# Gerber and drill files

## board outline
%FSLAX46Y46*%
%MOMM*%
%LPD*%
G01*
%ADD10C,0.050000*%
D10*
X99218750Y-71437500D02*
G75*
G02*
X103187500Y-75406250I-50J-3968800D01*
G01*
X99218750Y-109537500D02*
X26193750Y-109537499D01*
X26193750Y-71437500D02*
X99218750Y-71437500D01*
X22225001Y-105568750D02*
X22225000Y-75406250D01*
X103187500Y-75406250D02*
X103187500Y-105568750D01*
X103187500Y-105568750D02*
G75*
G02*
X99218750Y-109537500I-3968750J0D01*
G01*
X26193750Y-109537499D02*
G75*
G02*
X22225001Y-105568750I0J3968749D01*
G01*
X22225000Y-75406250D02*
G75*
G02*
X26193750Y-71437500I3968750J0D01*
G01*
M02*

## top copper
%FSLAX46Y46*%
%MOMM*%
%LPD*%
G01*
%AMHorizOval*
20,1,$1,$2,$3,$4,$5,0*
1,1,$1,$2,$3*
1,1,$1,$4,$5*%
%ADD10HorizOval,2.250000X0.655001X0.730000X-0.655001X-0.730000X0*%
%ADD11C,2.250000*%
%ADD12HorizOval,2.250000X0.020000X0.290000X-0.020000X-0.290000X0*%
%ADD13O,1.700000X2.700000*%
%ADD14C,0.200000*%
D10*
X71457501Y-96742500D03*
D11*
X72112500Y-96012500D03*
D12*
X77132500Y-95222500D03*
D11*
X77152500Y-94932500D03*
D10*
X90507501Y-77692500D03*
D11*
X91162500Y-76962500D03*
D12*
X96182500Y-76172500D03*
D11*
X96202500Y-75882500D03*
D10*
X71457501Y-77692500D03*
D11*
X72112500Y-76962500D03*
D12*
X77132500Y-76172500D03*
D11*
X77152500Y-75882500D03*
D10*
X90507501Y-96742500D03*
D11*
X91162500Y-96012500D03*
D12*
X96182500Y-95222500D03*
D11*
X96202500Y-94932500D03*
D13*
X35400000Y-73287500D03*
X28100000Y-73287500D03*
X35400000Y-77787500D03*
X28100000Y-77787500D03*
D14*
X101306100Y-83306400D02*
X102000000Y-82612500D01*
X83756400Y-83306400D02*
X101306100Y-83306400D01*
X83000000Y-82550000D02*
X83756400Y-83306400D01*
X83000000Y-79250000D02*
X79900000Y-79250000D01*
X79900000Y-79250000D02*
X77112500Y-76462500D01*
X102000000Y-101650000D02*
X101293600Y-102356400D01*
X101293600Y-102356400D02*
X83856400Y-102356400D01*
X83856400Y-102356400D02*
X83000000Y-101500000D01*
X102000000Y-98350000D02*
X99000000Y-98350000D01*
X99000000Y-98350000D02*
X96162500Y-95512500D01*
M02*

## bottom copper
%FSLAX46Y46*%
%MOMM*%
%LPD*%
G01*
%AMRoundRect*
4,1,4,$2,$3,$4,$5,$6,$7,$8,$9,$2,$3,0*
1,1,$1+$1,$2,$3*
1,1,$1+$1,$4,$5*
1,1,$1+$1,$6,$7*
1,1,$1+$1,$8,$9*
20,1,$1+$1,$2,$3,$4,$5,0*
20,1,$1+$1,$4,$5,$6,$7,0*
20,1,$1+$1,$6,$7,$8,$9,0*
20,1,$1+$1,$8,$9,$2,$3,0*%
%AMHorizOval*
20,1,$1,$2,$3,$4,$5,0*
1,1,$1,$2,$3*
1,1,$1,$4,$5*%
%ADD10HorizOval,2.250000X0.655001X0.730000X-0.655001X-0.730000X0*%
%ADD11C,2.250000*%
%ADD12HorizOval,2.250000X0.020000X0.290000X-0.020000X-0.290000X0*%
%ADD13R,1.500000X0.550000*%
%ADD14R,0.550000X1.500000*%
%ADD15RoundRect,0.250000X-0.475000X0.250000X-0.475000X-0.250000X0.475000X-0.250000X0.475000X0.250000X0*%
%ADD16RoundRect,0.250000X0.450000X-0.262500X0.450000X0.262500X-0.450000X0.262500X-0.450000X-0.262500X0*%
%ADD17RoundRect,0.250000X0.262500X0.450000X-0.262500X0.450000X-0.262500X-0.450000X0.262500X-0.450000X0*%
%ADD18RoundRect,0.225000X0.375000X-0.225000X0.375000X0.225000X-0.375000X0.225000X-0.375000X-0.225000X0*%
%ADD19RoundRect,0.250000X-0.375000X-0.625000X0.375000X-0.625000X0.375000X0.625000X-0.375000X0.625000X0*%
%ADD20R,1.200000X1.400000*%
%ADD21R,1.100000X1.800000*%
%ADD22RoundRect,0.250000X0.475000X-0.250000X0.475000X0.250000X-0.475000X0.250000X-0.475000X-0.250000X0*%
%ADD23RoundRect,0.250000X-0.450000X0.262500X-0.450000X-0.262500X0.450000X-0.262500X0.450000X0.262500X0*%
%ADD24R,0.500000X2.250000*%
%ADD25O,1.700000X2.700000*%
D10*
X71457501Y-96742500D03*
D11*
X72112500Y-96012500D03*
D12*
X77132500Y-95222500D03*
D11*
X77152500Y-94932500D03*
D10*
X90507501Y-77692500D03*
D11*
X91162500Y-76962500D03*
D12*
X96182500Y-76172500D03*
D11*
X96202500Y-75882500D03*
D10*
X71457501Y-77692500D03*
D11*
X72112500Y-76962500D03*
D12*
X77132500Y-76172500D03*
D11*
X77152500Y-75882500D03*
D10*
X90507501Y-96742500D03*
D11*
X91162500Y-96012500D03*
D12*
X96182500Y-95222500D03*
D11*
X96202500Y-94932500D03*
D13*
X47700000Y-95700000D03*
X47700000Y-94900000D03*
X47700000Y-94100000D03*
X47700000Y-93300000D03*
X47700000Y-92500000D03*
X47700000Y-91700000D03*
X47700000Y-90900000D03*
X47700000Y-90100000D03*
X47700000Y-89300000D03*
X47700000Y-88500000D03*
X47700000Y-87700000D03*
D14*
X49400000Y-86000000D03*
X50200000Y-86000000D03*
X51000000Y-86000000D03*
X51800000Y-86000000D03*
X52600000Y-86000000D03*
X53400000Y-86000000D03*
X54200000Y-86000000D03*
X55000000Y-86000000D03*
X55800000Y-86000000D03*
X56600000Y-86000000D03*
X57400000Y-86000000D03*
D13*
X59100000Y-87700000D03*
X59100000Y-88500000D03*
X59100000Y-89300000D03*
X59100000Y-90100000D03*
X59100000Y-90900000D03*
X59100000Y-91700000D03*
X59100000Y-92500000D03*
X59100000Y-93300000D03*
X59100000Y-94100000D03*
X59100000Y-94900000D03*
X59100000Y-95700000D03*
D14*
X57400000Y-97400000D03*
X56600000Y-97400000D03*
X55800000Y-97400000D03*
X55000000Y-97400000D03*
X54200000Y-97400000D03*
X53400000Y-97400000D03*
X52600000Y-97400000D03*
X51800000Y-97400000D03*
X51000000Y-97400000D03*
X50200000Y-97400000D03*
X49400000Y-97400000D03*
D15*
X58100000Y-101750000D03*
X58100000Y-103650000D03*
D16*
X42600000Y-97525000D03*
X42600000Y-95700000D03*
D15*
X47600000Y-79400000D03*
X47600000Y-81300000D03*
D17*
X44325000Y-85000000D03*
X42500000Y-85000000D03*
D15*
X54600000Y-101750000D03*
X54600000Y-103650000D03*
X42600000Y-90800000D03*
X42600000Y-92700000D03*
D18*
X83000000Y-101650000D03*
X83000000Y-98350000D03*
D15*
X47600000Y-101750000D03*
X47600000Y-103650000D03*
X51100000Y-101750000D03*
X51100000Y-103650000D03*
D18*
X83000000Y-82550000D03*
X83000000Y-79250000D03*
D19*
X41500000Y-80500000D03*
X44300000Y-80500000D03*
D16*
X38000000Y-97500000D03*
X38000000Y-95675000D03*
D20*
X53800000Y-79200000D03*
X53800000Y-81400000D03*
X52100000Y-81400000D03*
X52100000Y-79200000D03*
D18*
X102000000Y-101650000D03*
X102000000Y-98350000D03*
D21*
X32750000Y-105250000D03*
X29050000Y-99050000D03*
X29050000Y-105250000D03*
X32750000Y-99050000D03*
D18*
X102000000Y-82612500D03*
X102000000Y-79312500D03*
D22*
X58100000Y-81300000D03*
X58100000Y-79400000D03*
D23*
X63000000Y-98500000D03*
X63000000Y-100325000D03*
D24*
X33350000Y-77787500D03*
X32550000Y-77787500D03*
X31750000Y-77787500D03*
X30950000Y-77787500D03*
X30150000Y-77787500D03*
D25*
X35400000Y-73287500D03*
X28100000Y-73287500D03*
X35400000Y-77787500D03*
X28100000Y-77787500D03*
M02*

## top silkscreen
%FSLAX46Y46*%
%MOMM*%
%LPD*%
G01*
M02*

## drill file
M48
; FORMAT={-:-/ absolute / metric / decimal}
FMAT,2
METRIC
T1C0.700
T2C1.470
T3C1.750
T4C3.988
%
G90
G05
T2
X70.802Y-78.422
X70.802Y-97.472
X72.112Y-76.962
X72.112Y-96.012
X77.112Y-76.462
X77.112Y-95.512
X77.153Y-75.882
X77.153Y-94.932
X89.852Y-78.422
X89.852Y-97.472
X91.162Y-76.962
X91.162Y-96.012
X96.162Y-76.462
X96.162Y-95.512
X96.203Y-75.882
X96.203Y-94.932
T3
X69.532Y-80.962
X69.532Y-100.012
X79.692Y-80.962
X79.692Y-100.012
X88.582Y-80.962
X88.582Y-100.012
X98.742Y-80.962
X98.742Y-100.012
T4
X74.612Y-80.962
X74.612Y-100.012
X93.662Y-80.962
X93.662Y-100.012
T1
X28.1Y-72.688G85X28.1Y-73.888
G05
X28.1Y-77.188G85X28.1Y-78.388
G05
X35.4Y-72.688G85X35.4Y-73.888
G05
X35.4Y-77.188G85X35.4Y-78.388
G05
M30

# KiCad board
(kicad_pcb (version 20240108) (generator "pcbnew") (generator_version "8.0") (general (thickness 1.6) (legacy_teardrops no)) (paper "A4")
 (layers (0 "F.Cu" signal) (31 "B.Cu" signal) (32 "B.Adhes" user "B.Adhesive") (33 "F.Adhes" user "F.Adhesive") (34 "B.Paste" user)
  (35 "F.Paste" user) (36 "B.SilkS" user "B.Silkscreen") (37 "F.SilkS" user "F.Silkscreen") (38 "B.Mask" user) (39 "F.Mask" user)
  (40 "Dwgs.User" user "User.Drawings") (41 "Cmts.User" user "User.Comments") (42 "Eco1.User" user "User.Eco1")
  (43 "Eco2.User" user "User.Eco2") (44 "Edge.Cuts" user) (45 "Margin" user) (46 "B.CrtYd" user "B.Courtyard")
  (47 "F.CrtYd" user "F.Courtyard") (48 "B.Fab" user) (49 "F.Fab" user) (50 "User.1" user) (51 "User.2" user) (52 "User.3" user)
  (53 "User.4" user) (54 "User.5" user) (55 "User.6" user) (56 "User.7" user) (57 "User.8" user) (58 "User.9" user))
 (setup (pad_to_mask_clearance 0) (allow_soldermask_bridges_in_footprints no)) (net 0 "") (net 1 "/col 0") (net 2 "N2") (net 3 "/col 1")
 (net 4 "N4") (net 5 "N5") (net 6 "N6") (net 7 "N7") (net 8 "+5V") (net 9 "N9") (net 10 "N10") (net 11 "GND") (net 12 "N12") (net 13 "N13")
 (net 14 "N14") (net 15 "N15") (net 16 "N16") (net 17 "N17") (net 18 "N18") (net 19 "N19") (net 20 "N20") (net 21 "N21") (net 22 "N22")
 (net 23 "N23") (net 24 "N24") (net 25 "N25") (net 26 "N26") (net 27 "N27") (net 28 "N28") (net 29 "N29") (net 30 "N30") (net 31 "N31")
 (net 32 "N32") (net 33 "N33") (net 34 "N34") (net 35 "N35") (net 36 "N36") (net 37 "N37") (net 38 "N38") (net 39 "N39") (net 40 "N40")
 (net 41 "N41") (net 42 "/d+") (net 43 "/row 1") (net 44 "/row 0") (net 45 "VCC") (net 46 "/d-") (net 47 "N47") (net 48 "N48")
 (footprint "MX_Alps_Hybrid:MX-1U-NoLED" (layer "F.Cu") (at 74.6125 100.0125)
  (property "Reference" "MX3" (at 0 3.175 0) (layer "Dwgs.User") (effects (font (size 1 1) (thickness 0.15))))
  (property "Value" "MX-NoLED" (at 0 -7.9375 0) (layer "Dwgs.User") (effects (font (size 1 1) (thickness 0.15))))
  (pad "" np_thru_hole circle (at -5.08 0 48.0996) (size 1.75 1.75) (drill 1.75) (layers "*.Cu" "*.Mask"))
  (pad "" np_thru_hole circle (at 0 0) (size 3.9878 3.9878) (drill 3.9878) (layers "*.Cu" "*.Mask"))
  (pad "" np_thru_hole circle (at 5.08 0 48.0996) (size 1.75 1.75) (drill 1.75) (layers "*.Cu" "*.Mask"))
  (pad "1" thru_hole oval (at -3.81 -2.54 48.0996) (size 4.211556 2.25) (drill 1.47 (offset 0.980778 0)) (layers "*.Cu" "B.Mask")
   (remove_unused_layers no) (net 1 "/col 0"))
  (pad "1" thru_hole circle (at -2.5 -4) (size 2.25 2.25) (drill 1.47) (layers "*.Cu" "B.Mask") (remove_unused_layers no) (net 1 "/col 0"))
  (pad "2" thru_hole oval (at 2.5 -4.5 86.0548) (size 2.831378 2.25) (drill 1.47 (offset 0.290689 0)) (layers "*.Cu" "B.Mask")
   (remove_unused_layers no) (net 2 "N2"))
  (pad "2" thru_hole circle (at 2.54 -5.08) (size 2.25 2.25) (drill 1.47) (layers "*.Cu" "B.Mask") (remove_unused_layers no) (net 2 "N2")))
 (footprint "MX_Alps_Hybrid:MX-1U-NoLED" (layer "F.Cu") (at 93.6625 80.9625)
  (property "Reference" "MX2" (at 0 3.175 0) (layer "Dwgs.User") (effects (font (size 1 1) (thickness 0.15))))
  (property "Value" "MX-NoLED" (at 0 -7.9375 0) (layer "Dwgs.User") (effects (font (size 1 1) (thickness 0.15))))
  (pad "" np_thru_hole circle (at -5.08 0 48.0996) (size 1.75 1.75) (drill 1.75) (layers "*.Cu" "*.Mask"))
  (pad "" np_thru_hole circle (at 0 0) (size 3.9878 3.9878) (drill 3.9878) (layers "*.Cu" "*.Mask"))
  (pad "" np_thru_hole circle (at 5.08 0 48.0996) (size 1.75 1.75) (drill 1.75) (layers "*.Cu" "*.Mask"))
  (pad "1" thru_hole oval (at -3.81 -2.54 48.0996) (size 4.211556 2.25) (drill 1.47 (offset 0.980778 0)) (layers "*.Cu" "B.Mask")
   (remove_unused_layers no) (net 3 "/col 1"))
  (pad "1" thru_hole circle (at -2.5 -4) (size 2.25 2.25) (drill 1.47) (layers "*.Cu" "B.Mask") (remove_unused_layers no) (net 3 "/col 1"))
  (pad "2" thru_hole oval (at 2.5 -4.5 86.0548) (size 2.831378 2.25) (drill 1.47 (offset 0.290689 0)) (layers "*.Cu" "B.Mask")
   (remove_unused_layers no) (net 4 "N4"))
  (pad "2" thru_hole circle (at 2.54 -5.08) (size 2.25 2.25) (drill 1.47) (layers "*.Cu" "B.Mask") (remove_unused_layers no) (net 4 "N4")))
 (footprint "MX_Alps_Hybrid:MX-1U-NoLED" (layer "F.Cu") (at 74.6125 80.9625)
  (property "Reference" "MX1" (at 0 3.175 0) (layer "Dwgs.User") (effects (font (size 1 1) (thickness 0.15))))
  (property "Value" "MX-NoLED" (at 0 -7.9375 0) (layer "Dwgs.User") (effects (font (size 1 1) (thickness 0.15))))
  (pad "" np_thru_hole circle (at -5.08 0 48.0996) (size 1.75 1.75) (drill 1.75) (layers "*.Cu" "*.Mask"))
  (pad "" np_thru_hole circle (at 0 0) (size 3.9878 3.9878) (drill 3.9878) (layers "*.Cu" "*.Mask"))
  (pad "" np_thru_hole circle (at 5.08 0 48.0996) (size 1.75 1.75) (drill 1.75) (layers "*.Cu" "*.Mask"))
  (pad "1" thru_hole oval (at -3.81 -2.54 48.0996) (size 4.211556 2.25) (drill 1.47 (offset 0.980778 0)) (layers "*.Cu" "B.Mask")
   (remove_unused_layers no) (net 1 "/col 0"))
  (pad "1" thru_hole circle (at -2.5 -4) (size 2.25 2.25) (drill 1.47) (layers "*.Cu" "B.Mask") (remove_unused_layers no) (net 1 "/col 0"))
  (pad "2" thru_hole oval (at 2.5 -4.5 86.0548) (size 2.831378 2.25) (drill 1.47 (offset 0.290689 0)) (layers "*.Cu" "B.Mask")
   (remove_unused_layers no) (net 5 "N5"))
  (pad "2" thru_hole circle (at 2.54 -5.08) (size 2.25 2.25) (drill 1.47) (layers "*.Cu" "B.Mask") (remove_unused_layers no) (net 5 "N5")))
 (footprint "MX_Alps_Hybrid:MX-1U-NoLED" (layer "F.Cu") (at 93.6625 100.0125)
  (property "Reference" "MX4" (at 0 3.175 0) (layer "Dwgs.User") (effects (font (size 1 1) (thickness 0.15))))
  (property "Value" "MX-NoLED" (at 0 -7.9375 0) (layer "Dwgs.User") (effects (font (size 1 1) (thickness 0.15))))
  (pad "" np_thru_hole circle (at -5.08 0 48.0996) (size 1.75 1.75) (drill 1.75) (layers "*.Cu" "*.Mask"))
  (pad "" np_thru_hole circle (at 0 0) (size 3.9878 3.9878) (drill 3.9878) (layers "*.Cu" "*.Mask"))
  (pad "" np_thru_hole circle (at 5.08 0 48.0996) (size 1.75 1.75) (drill 1.75) (layers "*.Cu" "*.Mask"))
  (pad "1" thru_hole oval (at -3.81 -2.54 48.0996) (size 4.211556 2.25) (drill 1.47 (offset 0.980778 0)) (layers "*.Cu" "B.Mask")
   (remove_unused_layers no) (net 3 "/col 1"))
  (pad "1" thru_hole circle (at -2.5 -4) (size 2.25 2.25) (drill 1.47) (layers "*.Cu" "B.Mask") (remove_unused_layers no) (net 3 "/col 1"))
  (pad "2" thru_hole oval (at 2.5 -4.5 86.0548) (size 2.831378 2.25) (drill 1.47 (offset 0.290689 0)) (layers "*.Cu" "B.Mask")
   (remove_unused_layers no) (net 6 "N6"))
  (pad "2" thru_hole circle (at 2.54 -5.08) (size 2.25 2.25) (drill 1.47) (layers "*.Cu" "B.Mask") (remove_unused_layers no) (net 6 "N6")))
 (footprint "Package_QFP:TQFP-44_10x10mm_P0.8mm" (layer "B.Cu") (at 53.4 91.7)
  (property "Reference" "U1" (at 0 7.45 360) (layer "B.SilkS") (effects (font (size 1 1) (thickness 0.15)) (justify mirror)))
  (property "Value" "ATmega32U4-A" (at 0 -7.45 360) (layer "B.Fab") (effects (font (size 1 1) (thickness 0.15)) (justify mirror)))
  (pad "1" smd rect (at -5.7 4) (size 1.5 0.55) (layers "B.Cu" "B.Paste" "B.Mask") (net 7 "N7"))
  (pad "2" smd rect (at -5.7 3.2) (size 1.5 0.55) (layers "B.Cu" "B.Paste" "B.Mask") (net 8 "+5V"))
  (pad "3" smd rect (at -5.7 2.4) (size 1.5 0.55) (layers "B.Cu" "B.Paste" "B.Mask") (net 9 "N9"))
  (pad "4" smd rect (at -5.7 1.6) (size 1.5 0.55) (layers "B.Cu" "B.Paste" "B.Mask") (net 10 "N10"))
  (pad "5" smd rect (at -5.7 0.8) (size 1.5 0.55) (layers "B.Cu" "B.Paste" "B.Mask") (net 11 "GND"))
  (pad "6" smd rect (at -5.7 0) (size 1.5 0.55) (layers "B.Cu" "B.Paste" "B.Mask") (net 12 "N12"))
  (pad "7" smd rect (at -5.7 -0.8) (size 1.5 0.55) (layers "B.Cu" "B.Paste" "B.Mask") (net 8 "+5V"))
  (pad "8" smd rect (at -5.7 -1.6) (size 1.5 0.55) (layers "B.Cu" "B.Paste" "B.Mask") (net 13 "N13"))
  (pad "9" smd rect (at -5.7 -2.4) (size 1.5 0.55) (layers "B.Cu" "B.Paste" "B.Mask") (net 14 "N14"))
  (pad "10" smd rect (at -5.7 -3.2) (size 1.5 0.55) (layers "B.Cu" "B.Paste" "B.Mask") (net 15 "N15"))
  (pad "11" smd rect (at -5.7 -4) (size 1.5 0.55) (layers "B.Cu" "B.Paste" "B.Mask") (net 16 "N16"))
  (pad "12" smd rect (at -4 -5.7 270) (size 1.5 0.55) (layers "B.Cu" "B.Paste" "B.Mask") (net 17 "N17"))
  (pad "13" smd rect (at -3.2 -5.7 270) (size 1.5 0.55) (layers "B.Cu" "B.Paste" "B.Mask") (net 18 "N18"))
  (pad "14" smd rect (at -2.4 -5.7 270) (size 1.5 0.55) (layers "B.Cu" "B.Paste" "B.Mask") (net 8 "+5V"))
  (pad "15" smd rect (at -1.6 -5.7 270) (size 1.5 0.55) (layers "B.Cu" "B.Paste" "B.Mask") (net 11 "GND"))
  (pad "16" smd rect (at -0.8 -5.7 270) (size 1.5 0.55) (layers "B.Cu" "B.Paste" "B.Mask") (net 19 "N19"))
  (pad "17" smd rect (at 0 -5.7 270) (size 1.5 0.55) (layers "B.Cu" "B.Paste" "B.Mask") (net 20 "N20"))
  (pad "18" smd rect (at 0.8 -5.7 270) (size 1.5 0.55) (layers "B.Cu" "B.Paste" "B.Mask") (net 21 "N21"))
  (pad "19" smd rect (at 1.6 -5.7 270) (size 1.5 0.55) (layers "B.Cu" "B.Paste" "B.Mask") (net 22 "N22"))
  (pad "20" smd rect (at 2.4 -5.7 270) (size 1.5 0.55) (layers "B.Cu" "B.Paste" "B.Mask") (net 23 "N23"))
  (pad "21" smd rect (at 3.2 -5.7 270) (size 1.5 0.55) (layers "B.Cu" "B.Paste" "B.Mask") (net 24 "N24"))
  (pad "22" smd rect (at 4 -5.7 270) (size 1.5 0.55) (layers "B.Cu" "B.Paste" "B.Mask") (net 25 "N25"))
  (pad "23" smd rect (at 5.7 -4) (size 1.5 0.55) (layers "B.Cu" "B.Paste" "B.Mask") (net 11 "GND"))
  (pad "24" smd rect (at 5.7 -3.2) (size 1.5 0.55) (layers "B.Cu" "B.Paste" "B.Mask") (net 8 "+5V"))
  (pad "25" smd rect (at 5.7 -2.4) (size 1.5 0.55) (layers "B.Cu" "B.Paste" "B.Mask") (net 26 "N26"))
  (pad "26" smd rect (at 5.7 -1.6) (size 1.5 0.55) (layers "B.Cu" "B.Paste" "B.Mask") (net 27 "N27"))
  (pad "27" smd rect (at 5.7 -0.8) (size 1.5 0.55) (layers "B.Cu" "B.Paste" "B.Mask") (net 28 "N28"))
  (pad "28" smd rect (at 5.7 0) (size 1.5 0.55) (layers "B.Cu" "B.Paste" "B.Mask") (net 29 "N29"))
  (pad "29" smd rect (at 5.7 0.8) (size 1.5 0.55) (layers "B.Cu" "B.Paste" "B.Mask") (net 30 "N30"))
  (pad "30" smd rect (at 5.7 1.6) (size 1.5 0.55) (layers "B.Cu" "B.Paste" "B.Mask") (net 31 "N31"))
  (pad "31" smd rect (at 5.7 2.4) (size 1.5 0.55) (layers "B.Cu" "B.Paste" "B.Mask") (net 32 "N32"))
  (pad "32" smd rect (at 5.7 3.2) (size 1.5 0.55) (layers "B.Cu" "B.Paste" "B.Mask") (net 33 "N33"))
  (pad "33" smd rect (at 5.7 4) (size 1.5 0.55) (layers "B.Cu" "B.Paste" "B.Mask") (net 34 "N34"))
  (pad "34" smd rect (at 4 5.7 270) (size 1.5 0.55) (layers "B.Cu" "B.Paste" "B.Mask") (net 8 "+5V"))
  (pad "35" smd rect (at 3.2 5.7 270) (size 1.5 0.55) (layers "B.Cu" "B.Paste" "B.Mask") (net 11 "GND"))
  (pad "36" smd rect (at 2.4 5.7 270) (size 1.5 0.55) (layers "B.Cu" "B.Paste" "B.Mask") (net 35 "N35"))
  (pad "37" smd rect (at 1.6 5.7 270) (size 1.5 0.55) (layers "B.Cu" "B.Paste" "B.Mask") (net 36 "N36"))
  (pad "38" smd rect (at 0.8 5.7 270) (size 1.5 0.55) (layers "B.Cu" "B.Paste" "B.Mask") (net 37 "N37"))
  (pad "39" smd rect (at 0 5.7 270) (size 1.5 0.55) (layers "B.Cu" "B.Paste" "B.Mask") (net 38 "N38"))
  (pad "40" smd rect (at -0.8 5.7 270) (size 1.5 0.55) (layers "B.Cu" "B.Paste" "B.Mask") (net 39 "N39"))
  (pad "41" smd rect (at -1.6 5.7 270) (size 1.5 0.55) (layers "B.Cu" "B.Paste" "B.Mask") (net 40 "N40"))
  (pad "42" smd rect (at -2.4 5.7 270) (size 1.5 0.55) (layers "B.Cu" "B.Paste" "B.Mask") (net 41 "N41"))
  (pad "43" smd rect (at -3.2 5.7 270) (size 1.5 0.55) (layers "B.Cu" "B.Paste" "B.Mask") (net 11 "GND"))
  (pad "44" smd rect (at -4 5.7 270) (size 1.5 0.55) (layers "B.Cu" "B.Paste" "B.Mask") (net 8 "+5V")))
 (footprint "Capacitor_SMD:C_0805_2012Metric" (layer "B.Cu") (at 58.1 102.7 -90)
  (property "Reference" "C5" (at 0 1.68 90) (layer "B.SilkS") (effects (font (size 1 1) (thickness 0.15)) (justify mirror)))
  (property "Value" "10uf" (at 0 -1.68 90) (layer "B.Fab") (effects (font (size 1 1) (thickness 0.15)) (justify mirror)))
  (pad "1" smd roundrect (at -0.95 0 270) (size 1 1.45) (layers "B.Cu" "B.Paste" "B.Mask") (roundrect_rratio 0.25) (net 8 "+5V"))
  (pad "2" smd roundrect (at 0.95 0 270) (size 1 1.45) (layers "B.Cu" "B.Paste" "B.Mask") (roundrect_rratio 0.25) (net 11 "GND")))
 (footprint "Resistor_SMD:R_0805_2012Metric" (layer "B.Cu") (at 42.6 96.6125 90)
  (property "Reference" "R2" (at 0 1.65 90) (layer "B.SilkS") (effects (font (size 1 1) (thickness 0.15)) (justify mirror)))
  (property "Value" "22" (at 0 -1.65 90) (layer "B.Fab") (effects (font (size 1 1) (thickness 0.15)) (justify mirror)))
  (pad "1" smd roundrect (at -0.9125 0 90) (size 1.025 1.4) (layers "B.Cu" "B.Paste" "B.Mask") (roundrect_rratio 0.243902) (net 10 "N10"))
  (pad "2" smd roundrect (at 0.9125 0 90) (size 1.025 1.4) (layers "B.Cu" "B.Paste" "B.Mask") (roundrect_rratio 0.243902) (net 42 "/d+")))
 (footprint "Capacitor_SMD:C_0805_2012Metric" (layer "B.Cu") (at 47.6 80.35 -90)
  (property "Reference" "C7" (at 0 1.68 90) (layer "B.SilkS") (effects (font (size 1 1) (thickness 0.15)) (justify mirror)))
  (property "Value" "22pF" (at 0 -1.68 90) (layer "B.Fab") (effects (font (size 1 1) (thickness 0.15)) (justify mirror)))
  (pad "1" smd roundrect (at -0.95 0 270) (size 1 1.45) (layers "B.Cu" "B.Paste" "B.Mask") (roundrect_rratio 0.25) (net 11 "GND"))
  (pad "2" smd roundrect (at 0.95 0 270) (size 1 1.45) (layers "B.Cu" "B.Paste" "B.Mask") (roundrect_rratio 0.25) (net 19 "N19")))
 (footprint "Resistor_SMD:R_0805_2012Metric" (layer "B.Cu") (at 43.4125 85 180)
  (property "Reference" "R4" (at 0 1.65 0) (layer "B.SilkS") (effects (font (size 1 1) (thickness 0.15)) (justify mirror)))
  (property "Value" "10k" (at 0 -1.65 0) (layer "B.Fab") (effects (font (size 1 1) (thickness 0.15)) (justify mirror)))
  (pad "1" smd roundrect (at -0.9125 0 180) (size 1.025 1.4) (layers "B.Cu" "B.Paste" "B.Mask") (roundrect_rratio 0.243902) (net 8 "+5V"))
  (pad "2" smd roundrect (at 0.9125 0 180) (size 1.025 1.4) (layers "B.Cu" "B.Paste" "B.Mask") (roundrect_rratio 0.243902) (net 18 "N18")))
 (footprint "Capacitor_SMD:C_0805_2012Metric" (layer "B.Cu") (at 54.6 102.7 -90)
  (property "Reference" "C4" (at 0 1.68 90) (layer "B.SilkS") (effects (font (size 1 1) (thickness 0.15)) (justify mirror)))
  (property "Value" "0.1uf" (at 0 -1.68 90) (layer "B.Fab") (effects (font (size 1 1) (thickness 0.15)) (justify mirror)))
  (pad "1" smd roundrect (at -0.95 0 270) (size 1 1.45) (layers "B.Cu" "B.Paste" "B.Mask") (roundrect_rratio 0.25) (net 8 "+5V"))
  (pad "2" smd roundrect (at 0.95 0 270) (size 1 1.45) (layers "B.Cu" "B.Paste" "B.Mask") (roundrect_rratio 0.25) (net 11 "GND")))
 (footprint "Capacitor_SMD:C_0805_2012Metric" (layer "B.Cu") (at 42.6 91.75 -90)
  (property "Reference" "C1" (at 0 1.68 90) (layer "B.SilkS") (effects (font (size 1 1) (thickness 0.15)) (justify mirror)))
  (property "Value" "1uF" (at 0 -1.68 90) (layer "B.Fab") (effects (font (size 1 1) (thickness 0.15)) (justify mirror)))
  (pad "1" smd roundrect (at -0.95 0 270) (size 1 1.45) (layers "B.Cu" "B.Paste" "B.Mask") (roundrect_rratio 0.25) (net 12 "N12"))
  (pad "2" smd roundrect (at 0.95 0 270) (size 1 1.45) (layers "B.Cu" "B.Paste" "B.Mask") (roundrect_rratio 0.25) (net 11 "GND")))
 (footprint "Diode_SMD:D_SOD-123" (layer "B.Cu") (at 83 100 90)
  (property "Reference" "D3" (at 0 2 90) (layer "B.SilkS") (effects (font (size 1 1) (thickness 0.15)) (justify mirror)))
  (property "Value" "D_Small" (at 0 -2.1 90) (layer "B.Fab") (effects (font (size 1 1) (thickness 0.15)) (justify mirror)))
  (pad "1" smd roundrect (at -1.65 0 90) (size 0.9 1.2) (layers "B.Cu" "B.Paste" "B.Mask") (roundrect_rratio 0.25) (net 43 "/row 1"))
  (pad "2" smd roundrect (at 1.65 0 90) (size 0.9 1.2) (layers "B.Cu" "B.Paste" "B.Mask") (roundrect_rratio 0.25) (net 2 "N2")))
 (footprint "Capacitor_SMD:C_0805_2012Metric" (layer "B.Cu") (at 47.6 102.7 -90)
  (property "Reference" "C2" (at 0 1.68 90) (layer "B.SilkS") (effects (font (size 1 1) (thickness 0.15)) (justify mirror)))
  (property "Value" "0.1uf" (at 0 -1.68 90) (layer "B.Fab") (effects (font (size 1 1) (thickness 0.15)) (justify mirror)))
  (pad "1" smd roundrect (at -0.95 0 270) (size 1 1.45) (layers "B.Cu" "B.Paste" "B.Mask") (roundrect_rratio 0.25) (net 8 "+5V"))
  (pad "2" smd roundrect (at 0.95 0 270) (size 1 1.45) (layers "B.Cu" "B.Paste" "B.Mask") (roundrect_rratio 0.25) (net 11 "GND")))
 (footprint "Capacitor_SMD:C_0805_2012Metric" (layer "B.Cu") (at 51.1 102.7 -90)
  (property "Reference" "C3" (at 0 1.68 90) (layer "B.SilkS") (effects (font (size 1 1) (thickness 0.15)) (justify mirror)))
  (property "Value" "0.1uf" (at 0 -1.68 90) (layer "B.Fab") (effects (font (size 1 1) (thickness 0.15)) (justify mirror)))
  (pad "1" smd roundrect (at -0.95 0 270) (size 1 1.45) (layers "B.Cu" "B.Paste" "B.Mask") (roundrect_rratio 0.25) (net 8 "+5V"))
  (pad "2" smd roundrect (at 0.95 0 270) (size 1 1.45) (layers "B.Cu" "B.Paste" "B.Mask") (roundrect_rratio 0.25) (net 11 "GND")))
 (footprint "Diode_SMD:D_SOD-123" (layer "B.Cu") (at 83 80.9 90)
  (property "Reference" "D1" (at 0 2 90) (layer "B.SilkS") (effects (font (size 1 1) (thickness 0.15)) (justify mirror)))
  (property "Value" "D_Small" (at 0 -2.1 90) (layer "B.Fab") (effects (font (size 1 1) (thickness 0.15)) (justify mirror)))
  (pad "1" smd roundrect (at -1.65 0 90) (size 0.9 1.2) (layers "B.Cu" "B.Paste" "B.Mask") (roundrect_rratio 0.25) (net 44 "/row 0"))
  (pad "2" smd roundrect (at 1.65 0 90) (size 0.9 1.2) (layers "B.Cu" "B.Paste" "B.Mask") (roundrect_rratio 0.25) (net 5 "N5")))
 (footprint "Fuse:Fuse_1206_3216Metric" (layer "B.Cu") (at 42.9 80.5)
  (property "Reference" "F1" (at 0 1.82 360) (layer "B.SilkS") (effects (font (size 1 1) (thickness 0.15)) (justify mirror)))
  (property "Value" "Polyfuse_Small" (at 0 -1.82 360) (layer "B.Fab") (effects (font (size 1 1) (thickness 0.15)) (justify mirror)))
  (pad "1" smd roundrect (at -1.4 0) (size 1.25 1.75) (layers "B.Cu" "B.Paste" "B.Mask") (roundrect_rratio 0.2) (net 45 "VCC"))
  (pad "2" smd roundrect (at 1.4 0) (size 1.25 1.75) (layers "B.Cu" "B.Paste" "B.Mask") (roundrect_rratio 0.2) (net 8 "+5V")))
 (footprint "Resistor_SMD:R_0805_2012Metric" (layer "B.Cu") (at 38 96.5875 90)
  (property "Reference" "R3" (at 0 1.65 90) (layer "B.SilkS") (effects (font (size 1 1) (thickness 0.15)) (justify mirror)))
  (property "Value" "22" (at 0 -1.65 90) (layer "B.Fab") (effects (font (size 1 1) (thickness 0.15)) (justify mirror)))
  (pad "1" smd roundrect (at -0.9125 0 90) (size 1.025 1.4) (layers "B.Cu" "B.Paste" "B.Mask") (roundrect_rratio 0.243902) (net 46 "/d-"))
  (pad "2" smd roundrect (at 0.9125 0 90) (size 1.025 1.4) (layers "B.Cu" "B.Paste" "B.Mask") (roundrect_rratio 0.243902) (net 9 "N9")))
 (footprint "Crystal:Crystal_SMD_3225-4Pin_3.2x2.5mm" (layer "B.Cu") (at 52.95 80.3 -90)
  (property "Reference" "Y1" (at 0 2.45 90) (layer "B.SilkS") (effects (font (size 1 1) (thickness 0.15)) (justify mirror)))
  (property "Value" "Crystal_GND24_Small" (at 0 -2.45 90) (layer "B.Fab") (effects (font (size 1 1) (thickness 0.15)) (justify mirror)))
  (pad "1" smd rect (at -1.1 -0.85 270) (size 1.4 1.2) (layers "B.Cu" "B.Paste" "B.Mask") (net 20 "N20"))
  (pad "2" smd rect (at 1.1 -0.85 270) (size 1.4 1.2) (layers "B.Cu" "B.Paste" "B.Mask") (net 11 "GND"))
  (pad "3" smd rect (at 1.1 0.85 270) (size 1.4 1.2) (layers "B.Cu" "B.Paste" "B.Mask") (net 19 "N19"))
  (pad "4" smd rect (at -1.1 0.85 270) (size 1.4 1.2) (layers "B.Cu" "B.Paste" "B.Mask") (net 11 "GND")))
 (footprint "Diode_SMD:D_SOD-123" (layer "B.Cu") (at 102 100 90)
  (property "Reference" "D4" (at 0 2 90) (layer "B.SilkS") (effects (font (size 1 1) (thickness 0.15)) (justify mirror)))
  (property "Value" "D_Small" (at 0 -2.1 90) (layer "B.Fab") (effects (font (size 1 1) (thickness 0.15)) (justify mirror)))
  (pad "1" smd roundrect (at -1.65 0 90) (size 0.9 1.2) (layers "B.Cu" "B.Paste" "B.Mask") (roundrect_rratio 0.25) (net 43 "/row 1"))
  (pad "2" smd roundrect (at 1.65 0 90) (size 0.9 1.2) (layers "B.Cu" "B.Paste" "B.Mask") (roundrect_rratio 0.25) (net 6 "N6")))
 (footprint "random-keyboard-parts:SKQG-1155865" (layer "B.Cu") (at 30.9 102.15 -90)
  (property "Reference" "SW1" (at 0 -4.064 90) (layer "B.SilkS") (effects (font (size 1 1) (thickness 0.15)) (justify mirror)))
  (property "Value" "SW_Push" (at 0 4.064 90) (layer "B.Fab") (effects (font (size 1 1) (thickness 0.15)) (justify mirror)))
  (pad "1" smd rect (at 3.1 -1.85 270) (size 1.8 1.1) (layers "B.Cu" "B.Paste" "B.Mask") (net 11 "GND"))
  (pad "2" smd rect (at -3.1 1.85 270) (size 1.8 1.1) (layers "B.Cu" "B.Paste" "B.Mask") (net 18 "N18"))
  (pad "3" smd rect (at 3.1 1.85 270) (size 1.8 1.1) (layers "B.Cu" "B.Paste" "B.Mask"))
  (pad "4" smd rect (at -3.1 -1.85 270) (size 1.8 1.1) (layers "B.Cu" "B.Paste" "B.Mask")))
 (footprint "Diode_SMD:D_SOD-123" (layer "B.Cu") (at 102 80.9625 90)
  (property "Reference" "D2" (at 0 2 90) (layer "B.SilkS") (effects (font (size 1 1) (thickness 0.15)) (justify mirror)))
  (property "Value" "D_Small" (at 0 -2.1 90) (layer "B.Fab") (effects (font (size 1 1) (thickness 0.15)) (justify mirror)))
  (pad "1" smd roundrect (at -1.65 0 90) (size 0.9 1.2) (layers "B.Cu" "B.Paste" "B.Mask") (roundrect_rratio 0.25) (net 44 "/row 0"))
  (pad "2" smd roundrect (at 1.65 0 90) (size 0.9 1.2) (layers "B.Cu" "B.Paste" "B.Mask") (roundrect_rratio 0.25) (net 4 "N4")))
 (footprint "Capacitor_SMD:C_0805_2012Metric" (layer "B.Cu") (at 58.1 80.35 90)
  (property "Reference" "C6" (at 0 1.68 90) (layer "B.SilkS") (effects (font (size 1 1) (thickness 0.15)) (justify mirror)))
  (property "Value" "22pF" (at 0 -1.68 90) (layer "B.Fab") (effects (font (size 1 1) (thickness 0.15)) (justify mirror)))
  (pad "1" smd roundrect (at -0.95 0 90) (size 1 1.45) (layers "B.Cu" "B.Paste" "B.Mask") (roundrect_rratio 0.25) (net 11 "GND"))
  (pad "2" smd roundrect (at 0.95 0 90) (size 1 1.45) (layers "B.Cu" "B.Paste" "B.Mask") (roundrect_rratio 0.25) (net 20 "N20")))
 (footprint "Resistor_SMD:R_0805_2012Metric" (layer "B.Cu") (at 63 99.4125 -90)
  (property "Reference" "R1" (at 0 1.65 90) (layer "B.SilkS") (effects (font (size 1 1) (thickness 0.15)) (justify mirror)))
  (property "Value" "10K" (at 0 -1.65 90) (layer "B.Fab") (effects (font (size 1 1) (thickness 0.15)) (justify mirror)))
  (pad "1" smd roundrect (at -0.9125 0 270) (size 1.025 1.4) (layers "B.Cu" "B.Paste" "B.Mask") (roundrect_rratio 0.243902) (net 34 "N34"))
  (pad "2" smd roundrect (at 0.9125 0 270) (size 1.025 1.4) (layers "B.Cu" "B.Paste" "B.Mask") (roundrect_rratio 0.243902) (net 11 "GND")))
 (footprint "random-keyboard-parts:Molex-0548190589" (layer "B.Cu") (at 31.75 73.2875 -90)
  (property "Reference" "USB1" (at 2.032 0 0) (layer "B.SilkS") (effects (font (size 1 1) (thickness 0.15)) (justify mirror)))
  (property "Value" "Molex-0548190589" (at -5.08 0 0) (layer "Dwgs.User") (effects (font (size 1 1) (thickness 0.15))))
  (pad "1" smd rect (at 4.5 -1.6 270) (size 2.25 0.5) (layers "B.Cu" "B.Paste" "B.Mask") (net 11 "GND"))
  (pad "2" smd rect (at 4.5 -0.8 270) (size 2.25 0.5) (layers "B.Cu" "B.Paste" "B.Mask") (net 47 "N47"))
  (pad "3" smd rect (at 4.5 0 270) (size 2.25 0.5) (layers "B.Cu" "B.Paste" "B.Mask") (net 42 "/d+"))
  (pad "4" smd rect (at 4.5 0.8 270) (size 2.25 0.5) (layers "B.Cu" "B.Paste" "B.Mask") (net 46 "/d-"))
  (pad "5" smd rect (at 4.5 1.6 270) (size 2.25 0.5) (layers "B.Cu" "B.Paste" "B.Mask") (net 45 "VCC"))
  (pad "6" thru_hole oval (at 0 -3.65 270) (size 2.7 1.7) (drill oval 1.9 0.7) (layers "*.Cu" "*.Mask") (remove_unused_layers no)
   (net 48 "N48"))
  (pad "6" thru_hole oval (at 0 3.65 270) (size 2.7 1.7) (drill oval 1.9 0.7) (layers "*.Cu" "*.Mask") (remove_unused_layers no)
   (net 48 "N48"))
  (pad "6" thru_hole oval (at 4.5 -3.65 270) (size 2.7 1.7) (drill oval 1.9 0.7) (layers "*.Cu" "*.Mask") (remove_unused_layers no)
   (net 48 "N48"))
  (pad "6" thru_hole oval (at 4.5 3.65 270) (size 2.7 1.7) (drill oval 1.9 0.7) (layers "*.Cu" "*.Mask") (remove_unused_layers no)
   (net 48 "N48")))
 (gr_arc (start 99.21875 71.4375) (mid 102.02508 72.59992) (end 103.1875 75.40625) (stroke (width 0.05) (type default)) (layer "Edge.Cuts"))
 (gr_line (start 99.21875 109.5375) (end 26.19375 109.537499) (stroke (width 0.05) (type default)) (layer "Edge.Cuts"))
 (gr_line (start 26.19375 71.4375) (end 99.21875 71.4375) (stroke (width 0.05) (type default)) (layer "Edge.Cuts"))
 (gr_line (start 22.225001 105.56875) (end 22.225 75.40625) (stroke (width 0.05) (type default)) (layer "Edge.Cuts"))
 (gr_line (start 103.1875 75.40625) (end 103.1875 105.56875) (stroke (width 0.05) (type default)) (layer "Edge.Cuts"))
 (gr_arc (start 103.1875 105.56875) (mid 102.02508 108.37508) (end 99.21875 109.5375) (stroke (width 0.05) (type default))
  (layer "Edge.Cuts"))
 (gr_arc (start 26.19375 109.537499) (mid 23.387421 108.375079) (end 22.225001 105.56875) (stroke (width 0.05) (type default))
  (layer "Edge.Cuts"))
 (gr_arc (start 22.225 75.40625) (mid 23.38742 72.59992) (end 26.19375 71.4375) (stroke (width 0.05) (type default)) (layer "Edge.Cuts"))
 (segment (start 101.3061 83.3064) (end 102 82.6125) (width 0.2) (layer "F.Cu") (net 44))
 (segment (start 83.7564 83.3064) (end 101.3061 83.3064) (width 0.2) (layer "F.Cu") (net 44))
 (segment (start 83 82.55) (end 83.7564 83.3064) (width 0.2) (layer "F.Cu") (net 44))
 (segment (start 83 79.25) (end 79.9 79.25) (width 0.2) (layer "F.Cu") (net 5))
 (segment (start 79.9 79.25) (end 77.1125 76.4625) (width 0.2) (layer "F.Cu") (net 5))
 (segment (start 102 101.65) (end 101.2936 102.3564) (width 0.2) (layer "F.Cu") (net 43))
 (segment (start 101.2936 102.3564) (end 83.8564 102.3564) (width 0.2) (layer "F.Cu") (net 43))
 (segment (start 83.8564 102.3564) (end 83 101.5) (width 0.2) (layer "F.Cu") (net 43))
 (segment (start 102 98.35) (end 99 98.35) (width 0.2) (layer "F.Cu") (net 6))
 (segment (start 99 98.35) (end 96.1625 95.5125) (width 0.2) (layer "F.Cu") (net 6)))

